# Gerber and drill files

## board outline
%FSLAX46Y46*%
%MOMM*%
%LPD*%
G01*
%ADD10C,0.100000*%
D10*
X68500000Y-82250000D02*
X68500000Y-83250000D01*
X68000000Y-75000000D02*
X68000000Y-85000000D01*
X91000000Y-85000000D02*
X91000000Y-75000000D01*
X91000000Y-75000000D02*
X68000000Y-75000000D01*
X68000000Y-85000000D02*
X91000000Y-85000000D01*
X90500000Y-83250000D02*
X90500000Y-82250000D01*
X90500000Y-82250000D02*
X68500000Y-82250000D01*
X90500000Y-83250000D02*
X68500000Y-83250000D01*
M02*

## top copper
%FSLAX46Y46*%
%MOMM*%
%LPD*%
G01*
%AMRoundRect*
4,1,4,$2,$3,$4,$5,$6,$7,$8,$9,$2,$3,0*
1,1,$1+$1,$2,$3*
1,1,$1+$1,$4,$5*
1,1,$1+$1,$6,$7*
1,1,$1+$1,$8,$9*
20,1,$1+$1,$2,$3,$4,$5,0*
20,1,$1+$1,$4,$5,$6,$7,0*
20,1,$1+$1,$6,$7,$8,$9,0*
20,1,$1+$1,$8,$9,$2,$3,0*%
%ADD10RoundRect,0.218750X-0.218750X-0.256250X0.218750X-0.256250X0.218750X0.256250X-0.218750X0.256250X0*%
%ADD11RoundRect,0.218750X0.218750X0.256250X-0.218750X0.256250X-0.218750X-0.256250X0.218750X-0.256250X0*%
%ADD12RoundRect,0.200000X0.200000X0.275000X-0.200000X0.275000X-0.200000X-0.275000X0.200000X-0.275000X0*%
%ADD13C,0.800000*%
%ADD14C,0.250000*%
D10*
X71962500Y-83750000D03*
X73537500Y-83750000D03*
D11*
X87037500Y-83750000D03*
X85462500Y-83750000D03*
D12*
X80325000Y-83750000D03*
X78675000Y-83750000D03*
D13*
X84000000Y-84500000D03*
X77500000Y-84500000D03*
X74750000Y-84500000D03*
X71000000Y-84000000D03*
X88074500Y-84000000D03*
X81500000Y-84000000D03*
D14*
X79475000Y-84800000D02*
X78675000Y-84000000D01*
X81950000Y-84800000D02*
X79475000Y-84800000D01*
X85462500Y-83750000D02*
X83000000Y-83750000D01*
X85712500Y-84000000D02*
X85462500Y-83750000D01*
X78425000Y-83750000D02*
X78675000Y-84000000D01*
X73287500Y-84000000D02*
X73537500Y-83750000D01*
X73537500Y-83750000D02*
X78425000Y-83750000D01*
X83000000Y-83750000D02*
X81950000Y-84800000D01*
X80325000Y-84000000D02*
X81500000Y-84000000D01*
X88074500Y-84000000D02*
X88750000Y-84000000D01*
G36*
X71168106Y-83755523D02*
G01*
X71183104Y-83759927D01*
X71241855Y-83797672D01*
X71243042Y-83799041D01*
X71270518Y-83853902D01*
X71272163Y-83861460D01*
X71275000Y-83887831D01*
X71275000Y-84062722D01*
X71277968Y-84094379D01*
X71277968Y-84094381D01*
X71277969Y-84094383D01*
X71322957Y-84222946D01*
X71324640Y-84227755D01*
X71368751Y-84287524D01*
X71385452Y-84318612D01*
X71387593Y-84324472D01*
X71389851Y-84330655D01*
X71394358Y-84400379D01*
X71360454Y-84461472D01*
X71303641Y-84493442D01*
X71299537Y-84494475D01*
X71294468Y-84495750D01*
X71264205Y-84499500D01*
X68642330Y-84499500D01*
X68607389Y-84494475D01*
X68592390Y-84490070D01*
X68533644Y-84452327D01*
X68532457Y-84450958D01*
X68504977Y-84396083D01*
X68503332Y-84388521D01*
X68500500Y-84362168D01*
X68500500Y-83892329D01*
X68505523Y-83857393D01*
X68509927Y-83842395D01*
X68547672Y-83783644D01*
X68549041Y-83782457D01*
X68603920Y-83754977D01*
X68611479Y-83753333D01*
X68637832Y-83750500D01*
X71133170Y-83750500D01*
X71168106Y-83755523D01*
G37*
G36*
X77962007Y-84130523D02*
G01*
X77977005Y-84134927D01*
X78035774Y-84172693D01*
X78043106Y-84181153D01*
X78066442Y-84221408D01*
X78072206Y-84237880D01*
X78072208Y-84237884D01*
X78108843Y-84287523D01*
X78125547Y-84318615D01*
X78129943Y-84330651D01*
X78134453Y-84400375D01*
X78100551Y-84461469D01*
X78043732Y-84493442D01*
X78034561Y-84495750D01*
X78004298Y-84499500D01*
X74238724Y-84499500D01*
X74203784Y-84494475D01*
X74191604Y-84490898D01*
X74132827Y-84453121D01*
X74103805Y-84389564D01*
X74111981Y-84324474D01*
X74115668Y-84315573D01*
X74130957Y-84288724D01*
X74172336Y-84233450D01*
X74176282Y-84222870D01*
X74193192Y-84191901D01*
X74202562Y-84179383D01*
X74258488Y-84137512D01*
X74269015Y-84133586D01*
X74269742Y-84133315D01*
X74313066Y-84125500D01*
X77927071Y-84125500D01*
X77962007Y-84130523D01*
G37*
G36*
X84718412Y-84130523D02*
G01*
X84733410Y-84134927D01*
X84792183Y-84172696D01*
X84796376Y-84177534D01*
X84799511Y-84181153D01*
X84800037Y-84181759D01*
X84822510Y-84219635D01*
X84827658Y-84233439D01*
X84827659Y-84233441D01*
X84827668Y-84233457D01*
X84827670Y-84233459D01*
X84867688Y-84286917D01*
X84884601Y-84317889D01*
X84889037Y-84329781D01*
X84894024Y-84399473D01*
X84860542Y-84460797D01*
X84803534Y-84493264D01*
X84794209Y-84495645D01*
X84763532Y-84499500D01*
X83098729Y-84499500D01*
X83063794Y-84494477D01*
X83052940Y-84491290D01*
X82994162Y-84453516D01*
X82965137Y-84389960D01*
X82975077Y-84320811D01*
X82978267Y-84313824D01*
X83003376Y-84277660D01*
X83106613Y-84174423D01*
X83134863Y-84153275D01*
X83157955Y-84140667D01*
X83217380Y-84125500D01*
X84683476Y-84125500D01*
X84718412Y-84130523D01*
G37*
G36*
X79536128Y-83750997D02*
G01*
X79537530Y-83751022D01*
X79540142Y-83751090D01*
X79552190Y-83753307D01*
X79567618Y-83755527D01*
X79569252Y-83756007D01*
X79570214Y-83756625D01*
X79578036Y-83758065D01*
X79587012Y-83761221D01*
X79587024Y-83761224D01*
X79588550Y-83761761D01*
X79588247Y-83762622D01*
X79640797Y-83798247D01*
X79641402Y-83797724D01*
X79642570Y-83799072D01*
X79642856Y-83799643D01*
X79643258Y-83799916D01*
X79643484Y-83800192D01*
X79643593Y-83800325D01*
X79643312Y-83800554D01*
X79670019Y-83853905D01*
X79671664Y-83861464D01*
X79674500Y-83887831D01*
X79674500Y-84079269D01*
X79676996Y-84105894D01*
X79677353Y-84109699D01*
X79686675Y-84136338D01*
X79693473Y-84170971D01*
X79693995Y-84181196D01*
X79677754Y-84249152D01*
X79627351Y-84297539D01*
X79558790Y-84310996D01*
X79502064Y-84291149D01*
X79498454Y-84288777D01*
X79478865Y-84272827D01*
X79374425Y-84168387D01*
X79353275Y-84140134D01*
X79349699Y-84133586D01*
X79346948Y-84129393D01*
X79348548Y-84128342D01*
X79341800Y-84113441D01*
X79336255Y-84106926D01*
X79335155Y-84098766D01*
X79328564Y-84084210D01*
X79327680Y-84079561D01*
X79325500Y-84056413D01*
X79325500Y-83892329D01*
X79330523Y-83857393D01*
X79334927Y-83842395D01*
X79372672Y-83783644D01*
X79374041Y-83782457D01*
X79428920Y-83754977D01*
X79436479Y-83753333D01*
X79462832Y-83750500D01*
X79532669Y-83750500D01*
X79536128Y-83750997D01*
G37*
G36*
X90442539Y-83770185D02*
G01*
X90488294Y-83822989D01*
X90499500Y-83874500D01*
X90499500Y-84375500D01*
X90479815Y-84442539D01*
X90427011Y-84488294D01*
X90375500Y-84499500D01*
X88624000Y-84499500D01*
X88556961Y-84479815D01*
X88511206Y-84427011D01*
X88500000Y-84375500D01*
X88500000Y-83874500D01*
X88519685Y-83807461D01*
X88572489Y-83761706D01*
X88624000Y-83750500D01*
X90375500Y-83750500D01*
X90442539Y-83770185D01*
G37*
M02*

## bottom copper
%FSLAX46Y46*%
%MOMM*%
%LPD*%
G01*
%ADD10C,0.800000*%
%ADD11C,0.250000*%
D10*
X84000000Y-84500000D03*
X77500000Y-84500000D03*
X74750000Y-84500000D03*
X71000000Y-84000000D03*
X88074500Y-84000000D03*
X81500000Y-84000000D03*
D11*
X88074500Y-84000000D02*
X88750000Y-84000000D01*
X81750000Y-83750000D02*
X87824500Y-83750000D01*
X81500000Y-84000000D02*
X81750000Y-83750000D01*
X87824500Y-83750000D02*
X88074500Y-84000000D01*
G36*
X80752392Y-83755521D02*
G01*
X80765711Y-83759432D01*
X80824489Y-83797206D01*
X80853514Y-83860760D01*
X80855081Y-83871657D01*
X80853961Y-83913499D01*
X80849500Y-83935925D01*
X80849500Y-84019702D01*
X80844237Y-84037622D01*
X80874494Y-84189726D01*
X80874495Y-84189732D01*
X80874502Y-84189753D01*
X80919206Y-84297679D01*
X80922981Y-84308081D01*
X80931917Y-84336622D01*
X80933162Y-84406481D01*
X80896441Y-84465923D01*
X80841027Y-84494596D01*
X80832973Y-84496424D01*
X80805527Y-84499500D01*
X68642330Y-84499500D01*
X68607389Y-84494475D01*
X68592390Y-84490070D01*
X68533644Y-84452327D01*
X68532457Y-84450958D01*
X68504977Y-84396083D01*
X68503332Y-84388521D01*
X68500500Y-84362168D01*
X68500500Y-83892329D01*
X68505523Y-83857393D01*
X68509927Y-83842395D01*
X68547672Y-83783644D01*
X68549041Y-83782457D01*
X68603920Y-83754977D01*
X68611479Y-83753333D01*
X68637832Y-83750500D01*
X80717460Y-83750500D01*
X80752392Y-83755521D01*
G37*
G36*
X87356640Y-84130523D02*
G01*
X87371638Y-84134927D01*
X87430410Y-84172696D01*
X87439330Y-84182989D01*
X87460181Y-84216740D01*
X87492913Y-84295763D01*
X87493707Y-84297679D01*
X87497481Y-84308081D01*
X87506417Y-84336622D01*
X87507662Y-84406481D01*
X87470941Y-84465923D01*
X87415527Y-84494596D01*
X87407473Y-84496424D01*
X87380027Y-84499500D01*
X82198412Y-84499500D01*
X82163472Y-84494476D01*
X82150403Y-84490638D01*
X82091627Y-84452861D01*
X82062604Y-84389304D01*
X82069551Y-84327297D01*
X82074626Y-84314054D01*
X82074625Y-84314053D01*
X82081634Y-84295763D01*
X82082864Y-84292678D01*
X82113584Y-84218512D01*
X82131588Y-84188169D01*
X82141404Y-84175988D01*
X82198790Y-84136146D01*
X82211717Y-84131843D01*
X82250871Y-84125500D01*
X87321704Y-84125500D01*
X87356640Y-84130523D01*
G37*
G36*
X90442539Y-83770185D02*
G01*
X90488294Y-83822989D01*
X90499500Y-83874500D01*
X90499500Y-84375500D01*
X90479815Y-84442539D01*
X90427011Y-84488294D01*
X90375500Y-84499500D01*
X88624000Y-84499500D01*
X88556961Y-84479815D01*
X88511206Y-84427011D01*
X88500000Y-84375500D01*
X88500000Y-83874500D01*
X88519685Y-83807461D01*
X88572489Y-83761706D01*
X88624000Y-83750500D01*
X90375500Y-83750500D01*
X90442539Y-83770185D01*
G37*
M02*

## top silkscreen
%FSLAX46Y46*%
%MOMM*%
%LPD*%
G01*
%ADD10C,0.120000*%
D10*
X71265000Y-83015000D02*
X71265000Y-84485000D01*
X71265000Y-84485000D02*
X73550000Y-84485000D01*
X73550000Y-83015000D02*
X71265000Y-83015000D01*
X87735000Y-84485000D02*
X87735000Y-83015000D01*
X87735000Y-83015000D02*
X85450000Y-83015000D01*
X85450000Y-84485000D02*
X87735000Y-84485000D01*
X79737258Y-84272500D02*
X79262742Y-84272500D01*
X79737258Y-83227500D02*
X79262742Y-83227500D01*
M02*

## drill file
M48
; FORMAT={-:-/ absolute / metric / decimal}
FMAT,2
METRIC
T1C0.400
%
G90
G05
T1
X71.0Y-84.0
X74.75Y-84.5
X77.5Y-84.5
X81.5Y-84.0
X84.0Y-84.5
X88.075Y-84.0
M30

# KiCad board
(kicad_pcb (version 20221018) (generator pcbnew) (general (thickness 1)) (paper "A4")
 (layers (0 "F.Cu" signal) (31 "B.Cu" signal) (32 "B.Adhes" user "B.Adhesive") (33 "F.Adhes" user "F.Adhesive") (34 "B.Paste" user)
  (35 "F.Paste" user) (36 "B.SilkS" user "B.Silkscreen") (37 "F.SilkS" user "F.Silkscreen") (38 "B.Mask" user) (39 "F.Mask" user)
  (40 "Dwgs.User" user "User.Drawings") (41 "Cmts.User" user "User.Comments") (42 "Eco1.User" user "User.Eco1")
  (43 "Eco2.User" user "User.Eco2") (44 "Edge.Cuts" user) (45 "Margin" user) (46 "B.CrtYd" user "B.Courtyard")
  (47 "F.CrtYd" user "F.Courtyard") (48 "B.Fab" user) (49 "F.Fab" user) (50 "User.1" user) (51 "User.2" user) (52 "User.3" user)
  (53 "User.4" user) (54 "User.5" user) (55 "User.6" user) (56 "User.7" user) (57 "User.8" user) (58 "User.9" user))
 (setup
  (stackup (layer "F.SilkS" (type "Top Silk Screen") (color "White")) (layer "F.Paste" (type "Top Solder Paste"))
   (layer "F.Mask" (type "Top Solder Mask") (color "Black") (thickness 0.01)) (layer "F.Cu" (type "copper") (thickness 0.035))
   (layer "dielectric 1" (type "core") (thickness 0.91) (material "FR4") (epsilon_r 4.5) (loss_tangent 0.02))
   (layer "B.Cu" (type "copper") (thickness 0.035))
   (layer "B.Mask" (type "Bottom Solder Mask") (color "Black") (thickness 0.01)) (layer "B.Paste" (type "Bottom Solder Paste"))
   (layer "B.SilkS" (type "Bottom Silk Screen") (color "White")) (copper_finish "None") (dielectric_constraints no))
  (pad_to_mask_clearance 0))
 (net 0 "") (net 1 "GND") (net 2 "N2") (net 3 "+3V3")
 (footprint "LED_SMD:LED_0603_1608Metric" (layer "F.Cu") (at 72.75 83.75)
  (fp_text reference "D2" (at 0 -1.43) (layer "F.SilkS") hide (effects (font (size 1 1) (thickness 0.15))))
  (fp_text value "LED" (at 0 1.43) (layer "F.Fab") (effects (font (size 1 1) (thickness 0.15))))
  (fp_line (start -1.485 -0.735) (end -1.485 0.735) (stroke (width 0.12) (type solid)) (layer "F.SilkS"))
  (fp_line (start -1.485 0.735) (end 0.8 0.735) (stroke (width 0.12) (type solid)) (layer "F.SilkS"))
  (fp_line (start 0.8 -0.735) (end -1.485 -0.735) (stroke (width 0.12) (type solid)) (layer "F.SilkS"))
  (pad "1" smd roundrect (at -0.7875 0) (size 0.875 0.95) (layers "F.Cu" "F.Paste" "F.Mask") (roundrect_rratio 0.25) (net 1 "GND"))
  (pad "2" smd roundrect (at 0.7875 0) (size 0.875 0.95) (layers "F.Cu" "F.Paste" "F.Mask") (roundrect_rratio 0.25) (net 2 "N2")))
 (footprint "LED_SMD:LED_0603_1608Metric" (layer "F.Cu") (at 86.25 83.75 180)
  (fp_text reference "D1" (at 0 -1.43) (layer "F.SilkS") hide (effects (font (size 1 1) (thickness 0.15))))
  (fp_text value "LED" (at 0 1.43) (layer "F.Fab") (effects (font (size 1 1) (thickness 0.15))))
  (fp_line (start -1.485 -0.735) (end -1.485 0.735) (stroke (width 0.12) (type solid)) (layer "F.SilkS"))
  (fp_line (start -1.485 0.735) (end 0.8 0.735) (stroke (width 0.12) (type solid)) (layer "F.SilkS"))
  (fp_line (start 0.8 -0.735) (end -1.485 -0.735) (stroke (width 0.12) (type solid)) (layer "F.SilkS"))
  (pad "1" smd roundrect (at -0.7875 0 180) (size 0.875 0.95) (layers "F.Cu" "F.Paste" "F.Mask") (roundrect_rratio 0.25) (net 1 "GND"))
  (pad "2" smd roundrect (at 0.7875 0 180) (size 0.875 0.95) (layers "F.Cu" "F.Paste" "F.Mask") (roundrect_rratio 0.25) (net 2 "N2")))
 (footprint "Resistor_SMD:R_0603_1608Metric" (layer "F.Cu") (at 79.5 83.75 180)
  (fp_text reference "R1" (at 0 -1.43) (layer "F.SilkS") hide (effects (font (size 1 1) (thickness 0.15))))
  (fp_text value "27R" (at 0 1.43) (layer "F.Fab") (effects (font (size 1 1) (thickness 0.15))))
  (fp_line (start -0.237258 -0.5225) (end 0.237258 -0.5225) (stroke (width 0.12) (type solid)) (layer "F.SilkS"))
  (fp_line (start -0.237258 0.5225) (end 0.237258 0.5225) (stroke (width 0.12) (type solid)) (layer "F.SilkS"))
  (pad "1" smd roundrect (at -0.825 0 180) (size 0.8 0.95) (layers "F.Cu" "F.Paste" "F.Mask") (roundrect_rratio 0.25) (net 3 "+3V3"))
  (pad "2" smd roundrect (at 0.825 0 180) (size 0.8 0.95) (layers "F.Cu" "F.Paste" "F.Mask") (roundrect_rratio 0.25) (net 2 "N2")))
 (gr_line (start 68.5 82.25) (end 68.5 83.25) (stroke (width 0.1) (type default)) (layer "Edge.Cuts"))
 (gr_line (start 68 75) (end 68 85) (stroke (width 0.1) (type default)) (layer "Edge.Cuts"))
 (gr_line (start 91 85) (end 91 75) (stroke (width 0.1) (type default)) (layer "Edge.Cuts"))
 (gr_line (start 91 75) (end 68 75) (stroke (width 0.1) (type default)) (layer "Edge.Cuts"))
 (gr_line (start 68 85) (end 91 85) (stroke (width 0.1) (type default)) (layer "Edge.Cuts"))
 (gr_line (start 90.5 83.25) (end 90.5 82.25) (stroke (width 0.1) (type default)) (layer "Edge.Cuts"))
 (gr_line (start 90.5 82.25) (end 68.5 82.25) (stroke (width 0.1) (type default)) (layer "Edge.Cuts"))
 (gr_line (start 90.5 83.25) (end 68.5 83.25) (stroke (width 0.1) (type default)) (layer "Edge.Cuts"))
 (via (at 84 84.5) (size 0.8) (drill 0.4) (layers "F.Cu" "B.Cu") (free) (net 1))
 (via (at 77.5 84.5) (size 0.8) (drill 0.4) (layers "F.Cu" "B.Cu") (free) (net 1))
 (via (at 74.75 84.5) (size 0.8) (drill 0.4) (layers "F.Cu" "B.Cu") (free) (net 1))
 (via (at 71 84) (size 0.8) (drill 0.4) (layers "F.Cu" "B.Cu") (free) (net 1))
 (segment (start 79.475 84.8) (end 78.675 84) (width 0.25) (layer "F.Cu") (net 2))
 (segment (start 81.95 84.8) (end 79.475 84.8) (width 0.25) (layer "F.Cu") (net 2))
 (segment (start 85.4625 83.75) (end 83 83.75) (width 0.25) (layer "F.Cu") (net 2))
 (segment (start 85.7125 84) (end 85.4625 83.75) (width 0.25) (layer "F.Cu") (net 2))
 (segment (start 78.425 83.75) (end 78.675 84) (width 0.25) (layer "F.Cu") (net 2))
 (segment (start 73.2875 84) (end 73.5375 83.75) (width 0.25) (layer "F.Cu") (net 2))
 (segment (start 73.5375 83.75) (end 78.425 83.75) (width 0.25) (layer "F.Cu") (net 2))
 (segment (start 83 83.75) (end 81.95 84.8) (width 0.25) (layer "F.Cu") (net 2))
 (segment (start 80.325 84) (end 81.5 84) (width 0.25) (layer "F.Cu") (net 3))
 (segment (start 88.0745 84) (end 88.75 84) (width 0.25) (layer "F.Cu") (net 3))
 (via (at 88.0745 84) (size 0.8) (drill 0.4) (layers "F.Cu" "B.Cu") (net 3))
 (via (at 81.5 84) (size 0.8) (drill 0.4) (layers "F.Cu" "B.Cu") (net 3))
 (segment (start 88.0745 84) (end 88.75 84) (width 0.25) (layer "B.Cu") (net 3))
 (segment (start 81.75 83.75) (end 87.8245 83.75) (width 0.25) (layer "B.Cu") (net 3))
 (segment (start 81.5 84) (end 81.75 83.75) (width 0.25) (layer "B.Cu") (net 3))
 (segment (start 87.8245 83.75) (end 88.0745 84) (width 0.25) (layer "B.Cu") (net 3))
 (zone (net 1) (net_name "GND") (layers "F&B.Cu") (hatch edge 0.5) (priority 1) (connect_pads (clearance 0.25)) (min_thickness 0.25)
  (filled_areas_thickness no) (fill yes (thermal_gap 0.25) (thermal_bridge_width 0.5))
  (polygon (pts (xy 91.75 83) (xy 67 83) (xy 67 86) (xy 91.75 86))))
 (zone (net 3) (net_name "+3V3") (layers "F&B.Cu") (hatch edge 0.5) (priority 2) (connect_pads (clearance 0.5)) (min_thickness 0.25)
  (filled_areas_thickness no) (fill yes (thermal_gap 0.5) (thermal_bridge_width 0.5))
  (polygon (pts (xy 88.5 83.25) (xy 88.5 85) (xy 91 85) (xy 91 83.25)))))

